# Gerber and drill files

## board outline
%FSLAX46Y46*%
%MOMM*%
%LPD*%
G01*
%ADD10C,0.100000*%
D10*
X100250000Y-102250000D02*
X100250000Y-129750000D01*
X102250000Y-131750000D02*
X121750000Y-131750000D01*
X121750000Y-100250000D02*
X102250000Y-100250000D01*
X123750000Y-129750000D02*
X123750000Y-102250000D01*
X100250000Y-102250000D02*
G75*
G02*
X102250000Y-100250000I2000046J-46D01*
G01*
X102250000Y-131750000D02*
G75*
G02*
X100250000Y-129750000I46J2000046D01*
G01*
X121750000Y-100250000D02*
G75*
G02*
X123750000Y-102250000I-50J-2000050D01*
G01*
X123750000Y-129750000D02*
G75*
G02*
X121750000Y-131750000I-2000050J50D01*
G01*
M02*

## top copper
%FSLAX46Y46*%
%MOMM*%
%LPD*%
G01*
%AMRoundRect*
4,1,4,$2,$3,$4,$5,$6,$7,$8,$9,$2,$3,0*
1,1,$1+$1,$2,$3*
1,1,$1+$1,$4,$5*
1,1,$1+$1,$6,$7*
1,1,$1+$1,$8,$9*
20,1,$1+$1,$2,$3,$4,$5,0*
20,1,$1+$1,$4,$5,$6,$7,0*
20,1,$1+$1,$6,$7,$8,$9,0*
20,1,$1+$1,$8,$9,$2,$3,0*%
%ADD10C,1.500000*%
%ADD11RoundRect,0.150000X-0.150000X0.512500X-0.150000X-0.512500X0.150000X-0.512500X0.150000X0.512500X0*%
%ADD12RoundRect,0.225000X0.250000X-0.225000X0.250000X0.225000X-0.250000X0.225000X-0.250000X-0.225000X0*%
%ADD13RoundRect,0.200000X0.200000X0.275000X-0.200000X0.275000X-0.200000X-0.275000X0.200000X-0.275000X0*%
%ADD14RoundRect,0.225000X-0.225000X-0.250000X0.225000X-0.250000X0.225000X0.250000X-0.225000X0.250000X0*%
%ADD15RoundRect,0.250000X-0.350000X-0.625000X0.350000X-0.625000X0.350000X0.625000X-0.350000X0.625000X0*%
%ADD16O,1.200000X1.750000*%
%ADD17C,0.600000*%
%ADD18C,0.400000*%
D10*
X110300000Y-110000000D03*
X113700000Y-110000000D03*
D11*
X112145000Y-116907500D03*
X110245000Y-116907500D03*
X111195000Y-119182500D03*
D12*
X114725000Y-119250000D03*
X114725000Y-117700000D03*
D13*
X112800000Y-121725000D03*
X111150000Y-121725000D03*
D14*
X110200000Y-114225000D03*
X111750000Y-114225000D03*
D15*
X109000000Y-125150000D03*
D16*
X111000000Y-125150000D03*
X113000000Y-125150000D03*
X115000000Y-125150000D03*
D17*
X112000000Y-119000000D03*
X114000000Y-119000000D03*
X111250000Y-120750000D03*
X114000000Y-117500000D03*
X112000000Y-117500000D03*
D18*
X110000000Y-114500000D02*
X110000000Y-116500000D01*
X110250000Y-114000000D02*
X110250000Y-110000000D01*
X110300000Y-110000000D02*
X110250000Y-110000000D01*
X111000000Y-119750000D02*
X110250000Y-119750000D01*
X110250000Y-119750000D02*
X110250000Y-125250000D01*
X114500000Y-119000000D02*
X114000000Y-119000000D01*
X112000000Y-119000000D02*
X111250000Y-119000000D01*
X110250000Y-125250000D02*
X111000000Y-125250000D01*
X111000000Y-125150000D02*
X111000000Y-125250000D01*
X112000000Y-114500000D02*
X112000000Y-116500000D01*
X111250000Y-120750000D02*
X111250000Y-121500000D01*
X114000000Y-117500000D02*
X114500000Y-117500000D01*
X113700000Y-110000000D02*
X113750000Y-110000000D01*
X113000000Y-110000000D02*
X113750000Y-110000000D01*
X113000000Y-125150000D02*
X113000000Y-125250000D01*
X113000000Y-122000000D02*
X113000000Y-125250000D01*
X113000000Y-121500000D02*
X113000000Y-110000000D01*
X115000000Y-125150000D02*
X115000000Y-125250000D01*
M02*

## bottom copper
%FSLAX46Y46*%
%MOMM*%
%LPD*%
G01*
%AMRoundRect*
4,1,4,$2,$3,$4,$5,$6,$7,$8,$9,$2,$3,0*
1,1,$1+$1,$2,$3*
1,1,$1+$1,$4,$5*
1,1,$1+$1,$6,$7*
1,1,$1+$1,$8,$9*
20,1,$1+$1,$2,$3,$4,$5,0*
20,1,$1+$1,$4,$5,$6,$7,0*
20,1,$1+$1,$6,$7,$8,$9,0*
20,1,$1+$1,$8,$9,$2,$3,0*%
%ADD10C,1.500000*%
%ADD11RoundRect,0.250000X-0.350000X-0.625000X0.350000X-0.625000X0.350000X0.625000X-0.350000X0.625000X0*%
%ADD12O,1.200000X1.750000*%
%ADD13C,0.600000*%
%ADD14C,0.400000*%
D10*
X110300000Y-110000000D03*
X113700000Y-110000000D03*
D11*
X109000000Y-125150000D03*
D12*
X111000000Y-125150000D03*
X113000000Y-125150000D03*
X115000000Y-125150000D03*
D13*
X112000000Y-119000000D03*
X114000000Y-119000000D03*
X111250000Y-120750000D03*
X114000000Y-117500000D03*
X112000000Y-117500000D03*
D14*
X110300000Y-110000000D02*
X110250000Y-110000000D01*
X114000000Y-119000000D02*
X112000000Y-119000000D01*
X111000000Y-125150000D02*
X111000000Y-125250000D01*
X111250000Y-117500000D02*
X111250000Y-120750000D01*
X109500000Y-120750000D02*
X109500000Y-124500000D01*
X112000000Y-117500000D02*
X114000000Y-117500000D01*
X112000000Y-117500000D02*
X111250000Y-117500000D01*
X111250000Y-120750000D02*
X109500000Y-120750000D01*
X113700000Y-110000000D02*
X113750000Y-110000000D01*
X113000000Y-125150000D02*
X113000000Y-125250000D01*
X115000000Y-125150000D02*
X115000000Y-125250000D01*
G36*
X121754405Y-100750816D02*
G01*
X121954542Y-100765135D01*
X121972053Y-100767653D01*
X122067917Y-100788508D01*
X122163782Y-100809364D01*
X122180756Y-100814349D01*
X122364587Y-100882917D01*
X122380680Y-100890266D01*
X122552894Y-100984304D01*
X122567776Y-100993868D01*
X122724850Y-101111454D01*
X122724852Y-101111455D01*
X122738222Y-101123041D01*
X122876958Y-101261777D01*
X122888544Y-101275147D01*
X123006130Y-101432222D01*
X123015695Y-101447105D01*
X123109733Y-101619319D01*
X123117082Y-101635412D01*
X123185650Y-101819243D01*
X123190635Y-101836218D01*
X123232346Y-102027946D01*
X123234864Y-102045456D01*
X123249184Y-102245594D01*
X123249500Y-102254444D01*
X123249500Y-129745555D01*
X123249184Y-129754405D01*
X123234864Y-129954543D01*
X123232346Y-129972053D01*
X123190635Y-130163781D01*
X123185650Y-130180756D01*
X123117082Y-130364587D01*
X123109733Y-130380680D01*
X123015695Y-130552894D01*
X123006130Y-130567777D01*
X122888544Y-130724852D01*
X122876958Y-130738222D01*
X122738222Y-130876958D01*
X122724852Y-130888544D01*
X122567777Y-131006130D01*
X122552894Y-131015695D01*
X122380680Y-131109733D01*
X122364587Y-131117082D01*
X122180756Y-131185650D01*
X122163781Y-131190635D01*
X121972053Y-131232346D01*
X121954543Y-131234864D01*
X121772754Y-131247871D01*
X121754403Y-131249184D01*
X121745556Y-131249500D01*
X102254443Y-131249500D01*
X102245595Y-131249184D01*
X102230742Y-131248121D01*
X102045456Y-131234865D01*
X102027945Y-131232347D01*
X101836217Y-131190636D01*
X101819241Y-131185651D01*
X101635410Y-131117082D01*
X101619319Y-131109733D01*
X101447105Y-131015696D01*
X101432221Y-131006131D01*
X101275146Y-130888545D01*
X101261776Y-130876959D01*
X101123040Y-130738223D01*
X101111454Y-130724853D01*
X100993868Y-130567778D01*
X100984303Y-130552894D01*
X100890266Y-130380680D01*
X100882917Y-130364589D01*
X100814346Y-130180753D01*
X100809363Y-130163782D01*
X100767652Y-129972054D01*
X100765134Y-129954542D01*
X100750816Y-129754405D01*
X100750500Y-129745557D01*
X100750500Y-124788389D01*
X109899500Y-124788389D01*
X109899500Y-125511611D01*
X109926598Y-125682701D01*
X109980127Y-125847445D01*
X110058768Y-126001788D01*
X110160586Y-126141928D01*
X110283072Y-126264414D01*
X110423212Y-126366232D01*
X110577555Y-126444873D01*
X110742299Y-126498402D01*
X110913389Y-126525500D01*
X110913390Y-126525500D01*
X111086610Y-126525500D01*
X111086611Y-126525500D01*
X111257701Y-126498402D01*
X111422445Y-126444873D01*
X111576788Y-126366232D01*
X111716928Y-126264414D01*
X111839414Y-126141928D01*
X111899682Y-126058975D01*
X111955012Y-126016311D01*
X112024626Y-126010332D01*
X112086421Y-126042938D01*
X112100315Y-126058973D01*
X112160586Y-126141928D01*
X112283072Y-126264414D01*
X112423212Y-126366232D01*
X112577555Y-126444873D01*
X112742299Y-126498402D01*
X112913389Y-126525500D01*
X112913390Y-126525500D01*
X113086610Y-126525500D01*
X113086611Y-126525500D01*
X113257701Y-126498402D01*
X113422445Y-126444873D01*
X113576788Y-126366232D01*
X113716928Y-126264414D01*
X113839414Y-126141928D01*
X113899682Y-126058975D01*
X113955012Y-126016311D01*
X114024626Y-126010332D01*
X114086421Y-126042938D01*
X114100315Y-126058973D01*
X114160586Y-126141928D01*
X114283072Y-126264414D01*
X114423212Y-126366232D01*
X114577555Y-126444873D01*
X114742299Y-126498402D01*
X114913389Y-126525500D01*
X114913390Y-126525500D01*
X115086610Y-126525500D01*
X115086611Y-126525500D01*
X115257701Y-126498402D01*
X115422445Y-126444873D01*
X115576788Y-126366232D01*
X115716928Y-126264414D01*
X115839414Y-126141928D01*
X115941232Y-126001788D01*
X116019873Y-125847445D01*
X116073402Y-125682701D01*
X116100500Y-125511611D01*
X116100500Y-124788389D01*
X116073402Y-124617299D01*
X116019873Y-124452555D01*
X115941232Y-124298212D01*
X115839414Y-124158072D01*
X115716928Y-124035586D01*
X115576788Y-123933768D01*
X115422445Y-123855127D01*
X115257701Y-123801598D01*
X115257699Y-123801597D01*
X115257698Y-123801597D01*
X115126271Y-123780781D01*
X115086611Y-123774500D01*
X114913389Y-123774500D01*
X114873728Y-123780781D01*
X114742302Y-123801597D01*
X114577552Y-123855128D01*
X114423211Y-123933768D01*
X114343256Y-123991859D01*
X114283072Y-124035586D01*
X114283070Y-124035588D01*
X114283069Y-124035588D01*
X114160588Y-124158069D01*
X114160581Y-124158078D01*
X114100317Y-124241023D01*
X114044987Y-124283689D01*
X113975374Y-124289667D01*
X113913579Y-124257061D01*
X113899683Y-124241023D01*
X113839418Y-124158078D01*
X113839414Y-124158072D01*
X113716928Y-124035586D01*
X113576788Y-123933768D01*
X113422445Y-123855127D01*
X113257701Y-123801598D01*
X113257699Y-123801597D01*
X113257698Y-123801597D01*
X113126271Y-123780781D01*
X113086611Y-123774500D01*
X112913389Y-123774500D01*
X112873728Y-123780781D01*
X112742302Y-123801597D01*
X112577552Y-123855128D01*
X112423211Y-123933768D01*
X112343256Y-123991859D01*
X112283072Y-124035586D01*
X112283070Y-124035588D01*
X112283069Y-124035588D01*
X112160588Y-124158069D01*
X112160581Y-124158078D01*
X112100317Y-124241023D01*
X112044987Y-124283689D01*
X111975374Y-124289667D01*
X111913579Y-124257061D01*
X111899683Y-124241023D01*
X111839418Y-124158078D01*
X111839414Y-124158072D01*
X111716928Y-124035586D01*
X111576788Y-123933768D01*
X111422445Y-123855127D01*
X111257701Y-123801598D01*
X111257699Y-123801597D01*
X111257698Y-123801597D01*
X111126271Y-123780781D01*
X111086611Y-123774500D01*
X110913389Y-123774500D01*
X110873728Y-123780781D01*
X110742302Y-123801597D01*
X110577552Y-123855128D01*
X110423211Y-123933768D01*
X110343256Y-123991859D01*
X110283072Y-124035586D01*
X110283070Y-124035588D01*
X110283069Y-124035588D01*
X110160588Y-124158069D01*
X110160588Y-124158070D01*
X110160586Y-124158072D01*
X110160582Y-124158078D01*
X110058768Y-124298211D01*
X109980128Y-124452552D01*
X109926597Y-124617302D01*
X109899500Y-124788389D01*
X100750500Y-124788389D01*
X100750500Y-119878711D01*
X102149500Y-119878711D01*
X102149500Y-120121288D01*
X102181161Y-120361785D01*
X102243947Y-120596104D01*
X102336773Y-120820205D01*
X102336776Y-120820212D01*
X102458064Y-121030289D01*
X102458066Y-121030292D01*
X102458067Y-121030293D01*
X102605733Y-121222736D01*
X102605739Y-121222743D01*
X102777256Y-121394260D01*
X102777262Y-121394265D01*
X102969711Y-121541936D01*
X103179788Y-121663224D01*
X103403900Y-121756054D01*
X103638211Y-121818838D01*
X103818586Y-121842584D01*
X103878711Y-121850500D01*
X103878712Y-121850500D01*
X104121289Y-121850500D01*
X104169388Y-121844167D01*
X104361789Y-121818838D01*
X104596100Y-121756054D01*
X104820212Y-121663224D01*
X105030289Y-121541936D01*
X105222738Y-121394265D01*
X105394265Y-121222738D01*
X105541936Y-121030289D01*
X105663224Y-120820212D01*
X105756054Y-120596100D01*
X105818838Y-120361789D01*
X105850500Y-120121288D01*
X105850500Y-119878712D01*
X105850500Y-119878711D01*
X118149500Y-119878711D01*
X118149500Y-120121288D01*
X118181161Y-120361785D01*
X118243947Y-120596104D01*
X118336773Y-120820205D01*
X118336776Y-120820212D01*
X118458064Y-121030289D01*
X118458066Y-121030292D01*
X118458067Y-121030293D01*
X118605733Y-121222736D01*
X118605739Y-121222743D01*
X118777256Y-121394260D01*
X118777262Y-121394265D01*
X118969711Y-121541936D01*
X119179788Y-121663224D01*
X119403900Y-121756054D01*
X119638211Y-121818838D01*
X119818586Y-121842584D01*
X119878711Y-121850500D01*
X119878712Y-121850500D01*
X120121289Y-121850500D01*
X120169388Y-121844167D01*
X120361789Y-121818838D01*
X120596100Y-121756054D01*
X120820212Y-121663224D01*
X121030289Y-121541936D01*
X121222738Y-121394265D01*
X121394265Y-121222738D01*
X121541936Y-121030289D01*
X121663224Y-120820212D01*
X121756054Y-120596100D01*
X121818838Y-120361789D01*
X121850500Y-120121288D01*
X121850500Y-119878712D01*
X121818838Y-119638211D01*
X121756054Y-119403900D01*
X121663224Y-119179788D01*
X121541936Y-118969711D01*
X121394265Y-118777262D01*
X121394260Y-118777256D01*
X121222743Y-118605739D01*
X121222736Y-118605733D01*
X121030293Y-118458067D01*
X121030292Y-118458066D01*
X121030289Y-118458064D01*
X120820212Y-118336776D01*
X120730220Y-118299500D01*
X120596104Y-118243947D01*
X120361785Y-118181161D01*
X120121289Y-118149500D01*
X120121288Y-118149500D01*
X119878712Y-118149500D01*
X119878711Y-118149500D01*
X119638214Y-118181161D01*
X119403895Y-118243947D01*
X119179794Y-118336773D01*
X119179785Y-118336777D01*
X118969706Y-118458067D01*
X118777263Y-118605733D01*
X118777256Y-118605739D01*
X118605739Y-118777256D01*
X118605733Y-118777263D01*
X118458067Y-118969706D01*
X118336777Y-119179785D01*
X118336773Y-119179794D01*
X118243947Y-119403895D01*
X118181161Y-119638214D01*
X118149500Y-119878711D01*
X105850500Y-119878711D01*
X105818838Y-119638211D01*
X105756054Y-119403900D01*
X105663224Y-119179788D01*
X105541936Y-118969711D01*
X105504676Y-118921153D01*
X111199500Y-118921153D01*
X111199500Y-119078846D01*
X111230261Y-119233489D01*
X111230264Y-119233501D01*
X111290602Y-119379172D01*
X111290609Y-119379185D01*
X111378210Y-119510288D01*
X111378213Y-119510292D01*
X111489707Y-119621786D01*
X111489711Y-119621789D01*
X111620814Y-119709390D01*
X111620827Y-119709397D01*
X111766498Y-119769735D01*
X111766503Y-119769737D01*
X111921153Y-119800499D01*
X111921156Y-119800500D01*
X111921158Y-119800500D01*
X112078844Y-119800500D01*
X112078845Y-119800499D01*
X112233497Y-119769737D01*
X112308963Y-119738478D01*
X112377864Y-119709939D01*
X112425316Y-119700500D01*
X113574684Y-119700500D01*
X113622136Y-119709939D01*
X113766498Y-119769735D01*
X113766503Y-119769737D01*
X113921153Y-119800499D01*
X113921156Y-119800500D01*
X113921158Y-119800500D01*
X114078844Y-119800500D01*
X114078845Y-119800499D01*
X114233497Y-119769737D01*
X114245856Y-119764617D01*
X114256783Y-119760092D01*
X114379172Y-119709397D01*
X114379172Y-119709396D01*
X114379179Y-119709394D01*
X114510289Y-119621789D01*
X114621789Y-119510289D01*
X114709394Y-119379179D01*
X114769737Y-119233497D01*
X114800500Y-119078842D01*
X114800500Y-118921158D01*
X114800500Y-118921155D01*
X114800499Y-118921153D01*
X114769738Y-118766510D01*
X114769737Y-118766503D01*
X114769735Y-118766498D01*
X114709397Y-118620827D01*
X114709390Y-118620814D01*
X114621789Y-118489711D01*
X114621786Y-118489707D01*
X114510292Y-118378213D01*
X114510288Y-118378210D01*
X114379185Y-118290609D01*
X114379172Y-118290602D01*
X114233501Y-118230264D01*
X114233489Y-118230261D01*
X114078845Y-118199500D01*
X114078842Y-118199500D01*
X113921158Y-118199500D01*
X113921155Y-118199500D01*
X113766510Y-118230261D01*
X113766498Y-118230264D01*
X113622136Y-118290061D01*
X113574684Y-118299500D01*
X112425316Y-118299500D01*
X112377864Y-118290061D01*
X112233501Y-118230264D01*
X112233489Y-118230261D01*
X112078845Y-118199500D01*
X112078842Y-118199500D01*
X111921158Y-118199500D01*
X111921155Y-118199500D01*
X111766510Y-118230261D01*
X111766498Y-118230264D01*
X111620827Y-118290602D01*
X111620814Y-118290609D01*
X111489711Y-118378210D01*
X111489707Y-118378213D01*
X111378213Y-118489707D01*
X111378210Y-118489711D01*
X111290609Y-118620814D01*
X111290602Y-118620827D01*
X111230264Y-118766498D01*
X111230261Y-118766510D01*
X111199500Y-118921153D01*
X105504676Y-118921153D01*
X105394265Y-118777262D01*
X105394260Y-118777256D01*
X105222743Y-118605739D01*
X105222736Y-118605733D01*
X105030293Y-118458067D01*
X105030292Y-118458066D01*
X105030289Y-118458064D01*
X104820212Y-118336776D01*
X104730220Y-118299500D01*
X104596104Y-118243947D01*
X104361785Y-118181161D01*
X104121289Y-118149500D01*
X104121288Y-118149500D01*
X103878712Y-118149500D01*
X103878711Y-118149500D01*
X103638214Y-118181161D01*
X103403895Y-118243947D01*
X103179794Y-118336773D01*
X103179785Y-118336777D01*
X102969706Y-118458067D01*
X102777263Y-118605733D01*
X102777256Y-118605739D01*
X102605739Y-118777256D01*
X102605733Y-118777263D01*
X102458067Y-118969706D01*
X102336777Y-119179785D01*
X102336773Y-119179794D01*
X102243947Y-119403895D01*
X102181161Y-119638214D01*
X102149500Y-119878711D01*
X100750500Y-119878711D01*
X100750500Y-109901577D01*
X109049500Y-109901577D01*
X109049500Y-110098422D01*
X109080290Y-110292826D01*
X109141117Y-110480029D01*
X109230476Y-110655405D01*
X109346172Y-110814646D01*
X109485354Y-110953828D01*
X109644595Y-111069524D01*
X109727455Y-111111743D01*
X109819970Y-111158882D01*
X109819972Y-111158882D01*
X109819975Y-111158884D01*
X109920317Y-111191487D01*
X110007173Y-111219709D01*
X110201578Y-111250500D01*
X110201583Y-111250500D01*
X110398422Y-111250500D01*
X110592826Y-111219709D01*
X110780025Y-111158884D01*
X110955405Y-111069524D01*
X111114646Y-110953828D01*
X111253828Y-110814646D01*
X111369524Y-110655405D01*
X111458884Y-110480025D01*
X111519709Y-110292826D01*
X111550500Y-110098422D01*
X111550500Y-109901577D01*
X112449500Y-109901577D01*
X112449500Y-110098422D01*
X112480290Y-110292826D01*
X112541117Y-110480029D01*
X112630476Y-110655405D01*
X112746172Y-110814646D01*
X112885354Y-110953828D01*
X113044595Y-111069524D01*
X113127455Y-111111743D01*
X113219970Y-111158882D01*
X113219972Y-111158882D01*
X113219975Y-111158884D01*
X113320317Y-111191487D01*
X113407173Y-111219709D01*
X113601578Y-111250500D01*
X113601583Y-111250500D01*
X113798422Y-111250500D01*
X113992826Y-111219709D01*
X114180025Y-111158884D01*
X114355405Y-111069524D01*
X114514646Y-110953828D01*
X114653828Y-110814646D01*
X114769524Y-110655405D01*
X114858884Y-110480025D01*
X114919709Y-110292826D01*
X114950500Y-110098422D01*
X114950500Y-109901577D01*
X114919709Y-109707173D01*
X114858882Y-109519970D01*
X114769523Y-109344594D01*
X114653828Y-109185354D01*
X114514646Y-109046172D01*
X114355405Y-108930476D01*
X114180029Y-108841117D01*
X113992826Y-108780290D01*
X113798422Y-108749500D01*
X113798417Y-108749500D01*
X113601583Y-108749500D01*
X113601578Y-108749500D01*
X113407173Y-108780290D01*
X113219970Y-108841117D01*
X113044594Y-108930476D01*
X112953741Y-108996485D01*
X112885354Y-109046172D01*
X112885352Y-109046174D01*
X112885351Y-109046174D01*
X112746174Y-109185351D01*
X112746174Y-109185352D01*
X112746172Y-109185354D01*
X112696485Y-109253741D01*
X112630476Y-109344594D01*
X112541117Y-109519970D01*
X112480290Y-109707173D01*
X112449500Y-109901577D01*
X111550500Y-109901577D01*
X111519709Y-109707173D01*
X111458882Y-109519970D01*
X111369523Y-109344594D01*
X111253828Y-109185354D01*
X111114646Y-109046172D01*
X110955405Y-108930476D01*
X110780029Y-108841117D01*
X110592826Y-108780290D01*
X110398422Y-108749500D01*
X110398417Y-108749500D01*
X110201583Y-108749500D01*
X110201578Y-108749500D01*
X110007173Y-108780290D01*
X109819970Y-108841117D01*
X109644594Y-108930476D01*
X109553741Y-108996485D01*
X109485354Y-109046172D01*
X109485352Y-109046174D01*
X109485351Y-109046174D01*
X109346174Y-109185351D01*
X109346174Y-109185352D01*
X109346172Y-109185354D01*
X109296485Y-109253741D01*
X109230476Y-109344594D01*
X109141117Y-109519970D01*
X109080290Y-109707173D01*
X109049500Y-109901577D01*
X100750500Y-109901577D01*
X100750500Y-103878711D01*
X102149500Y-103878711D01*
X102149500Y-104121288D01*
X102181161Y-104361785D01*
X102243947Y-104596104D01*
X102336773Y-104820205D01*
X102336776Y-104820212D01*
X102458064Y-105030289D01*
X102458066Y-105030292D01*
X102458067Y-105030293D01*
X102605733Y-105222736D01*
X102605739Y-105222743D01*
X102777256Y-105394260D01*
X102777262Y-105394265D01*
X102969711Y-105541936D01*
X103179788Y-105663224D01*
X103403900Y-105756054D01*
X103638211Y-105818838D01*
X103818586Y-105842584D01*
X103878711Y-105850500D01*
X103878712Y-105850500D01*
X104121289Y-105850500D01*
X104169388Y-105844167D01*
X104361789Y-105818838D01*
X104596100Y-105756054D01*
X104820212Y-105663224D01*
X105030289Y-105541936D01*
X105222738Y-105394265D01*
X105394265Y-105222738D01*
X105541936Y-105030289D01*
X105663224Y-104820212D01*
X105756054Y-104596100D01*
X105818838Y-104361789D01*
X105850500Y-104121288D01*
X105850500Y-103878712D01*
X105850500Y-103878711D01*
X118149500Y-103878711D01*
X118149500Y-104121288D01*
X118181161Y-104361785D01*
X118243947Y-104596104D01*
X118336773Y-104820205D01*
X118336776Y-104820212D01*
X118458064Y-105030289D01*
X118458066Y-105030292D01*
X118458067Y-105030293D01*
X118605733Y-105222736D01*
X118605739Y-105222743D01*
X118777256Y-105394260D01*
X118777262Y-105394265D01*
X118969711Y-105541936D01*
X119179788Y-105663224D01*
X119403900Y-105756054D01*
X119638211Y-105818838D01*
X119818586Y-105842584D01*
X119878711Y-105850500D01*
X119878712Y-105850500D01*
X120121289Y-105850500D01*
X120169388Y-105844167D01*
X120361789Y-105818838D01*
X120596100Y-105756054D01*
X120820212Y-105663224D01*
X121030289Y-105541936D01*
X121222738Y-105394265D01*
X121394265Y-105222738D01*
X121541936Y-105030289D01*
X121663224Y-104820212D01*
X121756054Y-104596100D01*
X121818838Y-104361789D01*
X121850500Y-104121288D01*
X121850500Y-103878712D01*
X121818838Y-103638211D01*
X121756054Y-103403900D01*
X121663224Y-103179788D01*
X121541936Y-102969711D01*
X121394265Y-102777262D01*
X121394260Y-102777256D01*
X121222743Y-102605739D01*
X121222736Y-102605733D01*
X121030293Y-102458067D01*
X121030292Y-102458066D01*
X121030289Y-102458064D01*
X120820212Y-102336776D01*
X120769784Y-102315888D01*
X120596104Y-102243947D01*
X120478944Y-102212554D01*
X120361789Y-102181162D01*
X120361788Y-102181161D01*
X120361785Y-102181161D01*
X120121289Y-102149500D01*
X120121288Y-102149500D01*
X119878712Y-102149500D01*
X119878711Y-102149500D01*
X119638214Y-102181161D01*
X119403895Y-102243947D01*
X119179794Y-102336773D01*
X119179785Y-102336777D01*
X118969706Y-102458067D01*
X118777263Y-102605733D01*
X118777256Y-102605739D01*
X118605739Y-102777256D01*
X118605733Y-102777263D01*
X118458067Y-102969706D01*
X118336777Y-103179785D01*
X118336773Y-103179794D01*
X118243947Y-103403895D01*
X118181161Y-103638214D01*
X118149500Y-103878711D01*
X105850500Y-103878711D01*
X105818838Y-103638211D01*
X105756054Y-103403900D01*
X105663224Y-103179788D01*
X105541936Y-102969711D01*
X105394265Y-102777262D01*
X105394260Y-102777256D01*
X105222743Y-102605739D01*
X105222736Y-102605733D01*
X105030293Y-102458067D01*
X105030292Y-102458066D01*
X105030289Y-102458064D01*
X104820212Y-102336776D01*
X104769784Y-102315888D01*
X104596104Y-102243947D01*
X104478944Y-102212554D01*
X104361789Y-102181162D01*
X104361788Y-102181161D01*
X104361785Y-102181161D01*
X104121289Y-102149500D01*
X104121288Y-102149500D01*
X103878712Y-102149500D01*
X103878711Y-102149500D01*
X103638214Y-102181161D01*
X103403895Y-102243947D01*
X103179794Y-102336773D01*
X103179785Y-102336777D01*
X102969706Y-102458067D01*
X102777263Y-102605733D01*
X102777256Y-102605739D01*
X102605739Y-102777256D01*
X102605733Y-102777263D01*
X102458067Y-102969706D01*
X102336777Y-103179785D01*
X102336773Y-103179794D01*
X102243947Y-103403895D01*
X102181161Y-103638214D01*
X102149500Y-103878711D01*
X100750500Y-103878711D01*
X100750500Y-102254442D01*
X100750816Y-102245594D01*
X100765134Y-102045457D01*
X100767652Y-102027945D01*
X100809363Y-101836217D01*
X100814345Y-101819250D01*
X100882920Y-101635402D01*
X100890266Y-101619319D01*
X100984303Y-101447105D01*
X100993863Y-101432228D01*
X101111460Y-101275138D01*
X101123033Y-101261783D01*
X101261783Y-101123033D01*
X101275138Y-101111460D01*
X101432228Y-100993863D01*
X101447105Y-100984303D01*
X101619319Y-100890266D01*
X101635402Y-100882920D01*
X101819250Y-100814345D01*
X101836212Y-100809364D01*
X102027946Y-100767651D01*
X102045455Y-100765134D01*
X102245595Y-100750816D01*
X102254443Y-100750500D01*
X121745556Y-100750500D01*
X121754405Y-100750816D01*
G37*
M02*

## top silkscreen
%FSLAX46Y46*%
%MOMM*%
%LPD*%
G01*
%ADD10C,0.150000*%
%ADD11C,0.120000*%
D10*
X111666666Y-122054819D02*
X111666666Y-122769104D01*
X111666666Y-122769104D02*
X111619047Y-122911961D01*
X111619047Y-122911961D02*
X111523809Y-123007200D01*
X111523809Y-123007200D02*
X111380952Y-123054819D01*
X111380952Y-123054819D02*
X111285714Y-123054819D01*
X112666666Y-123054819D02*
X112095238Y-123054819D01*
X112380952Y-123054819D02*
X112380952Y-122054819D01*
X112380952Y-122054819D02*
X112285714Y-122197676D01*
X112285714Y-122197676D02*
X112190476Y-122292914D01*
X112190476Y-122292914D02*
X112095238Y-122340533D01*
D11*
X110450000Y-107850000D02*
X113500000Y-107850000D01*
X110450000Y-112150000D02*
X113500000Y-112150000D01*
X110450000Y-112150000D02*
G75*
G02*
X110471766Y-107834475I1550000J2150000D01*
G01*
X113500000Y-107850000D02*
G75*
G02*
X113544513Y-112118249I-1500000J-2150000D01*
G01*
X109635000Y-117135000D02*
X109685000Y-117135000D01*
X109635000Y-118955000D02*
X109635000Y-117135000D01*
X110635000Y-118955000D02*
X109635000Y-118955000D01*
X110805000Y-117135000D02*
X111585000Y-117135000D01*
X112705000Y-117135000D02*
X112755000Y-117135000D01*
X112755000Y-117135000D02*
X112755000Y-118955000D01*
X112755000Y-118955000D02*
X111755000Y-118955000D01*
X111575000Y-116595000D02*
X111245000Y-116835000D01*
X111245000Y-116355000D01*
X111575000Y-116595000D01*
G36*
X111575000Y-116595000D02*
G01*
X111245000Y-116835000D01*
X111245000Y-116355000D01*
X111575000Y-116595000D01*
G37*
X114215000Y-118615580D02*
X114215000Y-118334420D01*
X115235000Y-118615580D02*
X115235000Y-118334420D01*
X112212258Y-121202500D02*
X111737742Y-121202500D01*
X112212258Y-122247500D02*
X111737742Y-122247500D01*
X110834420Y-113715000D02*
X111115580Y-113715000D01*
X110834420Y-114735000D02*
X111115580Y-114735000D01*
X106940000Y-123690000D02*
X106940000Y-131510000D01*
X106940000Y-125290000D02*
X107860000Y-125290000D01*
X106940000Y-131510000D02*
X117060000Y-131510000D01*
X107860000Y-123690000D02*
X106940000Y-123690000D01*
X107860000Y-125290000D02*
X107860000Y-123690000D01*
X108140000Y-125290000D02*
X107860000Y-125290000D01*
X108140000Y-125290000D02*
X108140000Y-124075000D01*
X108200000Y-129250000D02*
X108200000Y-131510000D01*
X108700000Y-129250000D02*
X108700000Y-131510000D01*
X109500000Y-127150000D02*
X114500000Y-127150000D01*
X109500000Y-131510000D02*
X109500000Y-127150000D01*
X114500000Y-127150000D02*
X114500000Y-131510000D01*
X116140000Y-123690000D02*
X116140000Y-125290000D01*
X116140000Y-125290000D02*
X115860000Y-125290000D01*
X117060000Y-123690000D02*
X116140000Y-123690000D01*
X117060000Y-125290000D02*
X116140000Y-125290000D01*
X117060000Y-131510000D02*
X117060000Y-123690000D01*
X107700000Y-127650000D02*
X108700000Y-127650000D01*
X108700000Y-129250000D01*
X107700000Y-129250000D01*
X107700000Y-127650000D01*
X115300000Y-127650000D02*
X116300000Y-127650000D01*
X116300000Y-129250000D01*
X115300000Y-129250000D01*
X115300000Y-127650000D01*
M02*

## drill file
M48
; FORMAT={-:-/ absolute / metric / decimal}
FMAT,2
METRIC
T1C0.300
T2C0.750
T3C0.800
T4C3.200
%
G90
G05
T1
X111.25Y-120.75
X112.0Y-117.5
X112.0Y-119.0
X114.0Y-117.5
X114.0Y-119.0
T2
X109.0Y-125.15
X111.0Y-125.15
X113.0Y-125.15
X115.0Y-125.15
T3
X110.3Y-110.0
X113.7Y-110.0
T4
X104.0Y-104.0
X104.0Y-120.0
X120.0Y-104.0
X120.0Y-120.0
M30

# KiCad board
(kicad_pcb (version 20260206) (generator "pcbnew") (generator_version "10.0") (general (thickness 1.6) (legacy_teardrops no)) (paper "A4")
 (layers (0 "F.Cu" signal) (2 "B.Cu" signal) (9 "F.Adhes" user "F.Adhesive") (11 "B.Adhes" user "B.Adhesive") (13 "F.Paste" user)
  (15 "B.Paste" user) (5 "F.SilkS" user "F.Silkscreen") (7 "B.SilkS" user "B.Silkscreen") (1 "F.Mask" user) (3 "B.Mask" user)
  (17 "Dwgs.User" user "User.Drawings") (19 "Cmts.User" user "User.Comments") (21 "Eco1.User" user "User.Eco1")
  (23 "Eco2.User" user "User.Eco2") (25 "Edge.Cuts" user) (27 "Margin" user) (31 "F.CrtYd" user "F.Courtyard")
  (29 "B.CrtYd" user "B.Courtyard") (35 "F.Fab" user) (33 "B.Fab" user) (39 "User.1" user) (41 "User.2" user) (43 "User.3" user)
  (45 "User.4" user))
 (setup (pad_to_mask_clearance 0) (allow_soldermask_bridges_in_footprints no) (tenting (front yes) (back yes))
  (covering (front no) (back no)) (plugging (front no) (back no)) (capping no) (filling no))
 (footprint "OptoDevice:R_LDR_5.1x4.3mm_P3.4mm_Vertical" (layer "F.Cu") (at 110.3 110)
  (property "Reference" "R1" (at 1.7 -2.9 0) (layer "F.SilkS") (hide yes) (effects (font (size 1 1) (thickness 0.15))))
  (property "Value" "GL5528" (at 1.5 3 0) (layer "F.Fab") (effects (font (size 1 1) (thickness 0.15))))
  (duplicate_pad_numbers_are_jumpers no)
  (fp_line (start 0.15 -2.15) (end 3.2 -2.15) (stroke (width 0.12) (type solid)) (layer "F.SilkS"))
  (fp_line (start 0.15 2.15) (end 3.2 2.15) (stroke (width 0.12) (type solid)) (layer "F.SilkS"))
  (fp_arc (start 0.15 2.15) (mid -0.950438 -0.013368) (end 0.171766 -2.165525) (stroke (width 0.12) (type solid)) (layer "F.SilkS"))
  (fp_arc (start 3.2 -2.15) (mid 4.321403 -0.027338) (end 3.244513 2.118249) (stroke (width 0.12) (type solid)) (layer "F.SilkS"))
  (pad "1" thru_hole circle (at 0 0) (size 1.5 1.5) (drill 0.8) (layers "*.Cu" "*.Mask") (remove_unused_layers no) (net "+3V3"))
  (pad "2" thru_hole circle (at 3.4 0) (size 1.5 1.5) (drill 0.8) (layers "*.Cu" "*.Mask") (remove_unused_layers no) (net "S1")))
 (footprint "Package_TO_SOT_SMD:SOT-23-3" (layer "F.Cu") (at 111.195 118.045 -90)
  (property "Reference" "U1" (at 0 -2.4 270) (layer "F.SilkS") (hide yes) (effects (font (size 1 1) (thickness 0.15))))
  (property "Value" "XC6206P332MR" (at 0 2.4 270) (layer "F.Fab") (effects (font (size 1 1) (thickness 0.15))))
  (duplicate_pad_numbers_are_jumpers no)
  (fp_line (start -0.91 1.56) (end -0.91 1.51) (stroke (width 0.12) (type solid)) (layer "F.SilkS"))
  (fp_line (start 0.91 1.56) (end -0.91 1.56) (stroke (width 0.12) (type solid)) (layer "F.SilkS"))
  (fp_line (start 0.91 0.56) (end 0.91 1.56) (stroke (width 0.12) (type solid)) (layer "F.SilkS"))
  (fp_line (start -0.91 0.39) (end -0.91 -0.39) (stroke (width 0.12) (type solid)) (layer "F.SilkS"))
  (fp_line (start -0.91 -1.51) (end -0.91 -1.56) (stroke (width 0.12) (type solid)) (layer "F.SilkS"))
  (fp_line (start -0.91 -1.56) (end 0.91 -1.56) (stroke (width 0.12) (type solid)) (layer "F.SilkS"))
  (fp_line (start 0.91 -1.56) (end 0.91 -0.56) (stroke (width 0.12) (type solid)) (layer "F.SilkS"))
  (fp_poly (pts (xy -1.45 -0.38) (xy -1.21 -0.05) (xy -1.69 -0.05)) (stroke (width 0.12) (type solid)) (fill yes) (layer "F.SilkS"))
  (pad "1" smd roundrect (at -1.1375 -0.95 270) (size 1.325 0.6) (layers "F.Cu" "F.Mask" "F.Paste") (roundrect_rratio 0.25) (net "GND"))
  (pad "2" smd roundrect (at -1.1375 0.95 270) (size 1.325 0.6) (layers "F.Cu" "F.Mask" "F.Paste") (roundrect_rratio 0.25) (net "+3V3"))
  (pad "3" smd roundrect (at 1.1375 0 270) (size 1.325 0.6) (layers "F.Cu" "F.Mask" "F.Paste") (roundrect_rratio 0.25) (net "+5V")))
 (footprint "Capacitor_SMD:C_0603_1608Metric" (layer "F.Cu") (at 114.725 118.475 90)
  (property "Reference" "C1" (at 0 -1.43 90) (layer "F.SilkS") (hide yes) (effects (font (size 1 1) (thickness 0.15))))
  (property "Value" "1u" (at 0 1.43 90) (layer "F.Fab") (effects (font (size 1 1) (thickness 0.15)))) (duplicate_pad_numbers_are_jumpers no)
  (fp_line (start -0.14058 -0.51) (end 0.14058 -0.51) (stroke (width 0.12) (type solid)) (layer "F.SilkS"))
  (fp_line (start -0.14058 0.51) (end 0.14058 0.51) (stroke (width 0.12) (type solid)) (layer "F.SilkS"))
  (pad "1" smd roundrect (at -0.775 0 90) (size 0.9 0.95) (layers "F.Cu" "F.Mask" "F.Paste") (roundrect_rratio 0.25) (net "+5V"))
  (pad "2" smd roundrect (at 0.775 0 90) (size 0.9 0.95) (layers "F.Cu" "F.Mask" "F.Paste") (roundrect_rratio 0.25) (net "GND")))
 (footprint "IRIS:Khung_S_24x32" (layer "F.Cu") (at 100 132)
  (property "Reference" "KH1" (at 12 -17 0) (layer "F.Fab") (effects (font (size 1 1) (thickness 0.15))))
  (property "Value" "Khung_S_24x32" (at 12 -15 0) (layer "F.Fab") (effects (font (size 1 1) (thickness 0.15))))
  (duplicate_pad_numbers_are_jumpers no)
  (fp_line (start 0.25 -29.75) (end 0.25 -2.25) (stroke (width 0.1) (type solid)) (layer "Edge.Cuts"))
  (fp_line (start 2.25 -0.25) (end 21.75 -0.25) (stroke (width 0.1) (type solid)) (layer "Edge.Cuts"))
  (fp_line (start 21.75 -31.75) (end 2.25 -31.75) (stroke (width 0.1) (type solid)) (layer "Edge.Cuts"))
  (fp_line (start 23.75 -2.25) (end 23.75 -29.75) (stroke (width 0.1) (type solid)) (layer "Edge.Cuts"))
  (fp_arc (start 0.25 -29.75) (mid 0.8358 -31.1642) (end 2.25 -31.75) (stroke (width 0.1) (type solid)) (layer "Edge.Cuts"))
  (fp_arc (start 2.25 -0.25) (mid 0.8358 -0.8358) (end 0.25 -2.25) (stroke (width 0.1) (type solid)) (layer "Edge.Cuts"))
  (fp_arc (start 21.75 -31.75) (mid 23.164199 -31.164199) (end 23.75 -29.75) (stroke (width 0.1) (type solid)) (layer "Edge.Cuts"))
  (fp_arc (start 23.75 -2.25) (mid 23.164199 -0.835801) (end 21.75 -0.25) (stroke (width 0.1) (type solid)) (layer "Edge.Cuts"))
  (pad "" np_thru_hole circle (at 4 -28) (size 3.2 3.2) (drill 3.2) (layers "*.Cu" "*.Mask"))
  (pad "" np_thru_hole circle (at 4 -12) (size 3.2 3.2) (drill 3.2) (layers "*.Cu" "*.Mask"))
  (pad "" np_thru_hole circle (at 20 -28) (size 3.2 3.2) (drill 3.2) (layers "*.Cu" "*.Mask"))
  (pad "" np_thru_hole circle (at 20 -12) (size 3.2 3.2) (drill 3.2) (layers "*.Cu" "*.Mask")))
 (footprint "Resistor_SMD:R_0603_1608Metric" (layer "F.Cu") (at 111.975 121.725 180)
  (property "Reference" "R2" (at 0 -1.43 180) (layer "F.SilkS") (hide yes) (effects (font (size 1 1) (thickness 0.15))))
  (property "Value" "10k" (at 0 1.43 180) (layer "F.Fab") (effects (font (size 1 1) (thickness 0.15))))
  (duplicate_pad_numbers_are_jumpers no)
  (fp_line (start -0.237258 0.5225) (end 0.237258 0.5225) (stroke (width 0.12) (type solid)) (layer "F.SilkS"))
  (fp_line (start -0.237258 -0.5225) (end 0.237258 -0.5225) (stroke (width 0.12) (type solid)) (layer "F.SilkS"))
  (pad "1" smd roundrect (at -0.825 0 180) (size 0.8 0.95) (layers "F.Cu" "F.Mask" "F.Paste") (roundrect_rratio 0.25) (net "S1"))
  (pad "2" smd roundrect (at 0.825 0 180) (size 0.8 0.95) (layers "F.Cu" "F.Mask" "F.Paste") (roundrect_rratio 0.25) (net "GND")))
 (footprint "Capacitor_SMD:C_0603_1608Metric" (layer "F.Cu") (at 110.975 114.225)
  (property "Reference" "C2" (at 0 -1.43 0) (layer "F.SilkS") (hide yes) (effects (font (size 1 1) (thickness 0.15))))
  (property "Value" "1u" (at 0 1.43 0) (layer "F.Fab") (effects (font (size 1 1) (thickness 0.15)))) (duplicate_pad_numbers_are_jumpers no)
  (fp_line (start -0.14058 -0.51) (end 0.14058 -0.51) (stroke (width 0.12) (type solid)) (layer "F.SilkS"))
  (fp_line (start -0.14058 0.51) (end 0.14058 0.51) (stroke (width 0.12) (type solid)) (layer "F.SilkS"))
  (pad "1" smd roundrect (at -0.775 0) (size 0.9 0.95) (layers "F.Cu" "F.Mask" "F.Paste") (roundrect_rratio 0.25) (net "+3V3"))
  (pad "2" smd roundrect (at 0.775 0) (size 0.9 0.95) (layers "F.Cu" "F.Mask" "F.Paste") (roundrect_rratio 0.25) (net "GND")))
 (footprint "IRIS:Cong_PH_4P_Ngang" (layer "F.Cu") (at 109 125.15)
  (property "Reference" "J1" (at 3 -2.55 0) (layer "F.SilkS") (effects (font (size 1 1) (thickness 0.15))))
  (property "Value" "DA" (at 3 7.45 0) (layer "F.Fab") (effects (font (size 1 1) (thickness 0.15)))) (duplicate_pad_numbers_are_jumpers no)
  (fp_line (start -2.06 -1.46) (end -2.06 6.36) (stroke (width 0.12) (type solid)) (layer "F.SilkS"))
  (fp_line (start -2.06 0.14) (end -1.14 0.14) (stroke (width 0.12) (type solid)) (layer "F.SilkS"))
  (fp_line (start -2.06 6.36) (end 8.06 6.36) (stroke (width 0.12) (type solid)) (layer "F.SilkS"))
  (fp_line (start -1.14 -1.46) (end -2.06 -1.46) (stroke (width 0.12) (type solid)) (layer "F.SilkS"))
  (fp_line (start -1.14 0.14) (end -1.14 -1.46) (stroke (width 0.12) (type solid)) (layer "F.SilkS"))
  (fp_line (start -0.86 0.14) (end -1.14 0.14) (stroke (width 0.12) (type solid)) (layer "F.SilkS"))
  (fp_line (start -0.86 0.14) (end -0.86 -1.075) (stroke (width 0.12) (type solid)) (layer "F.SilkS"))
  (fp_line (start -0.8 4.1) (end -0.8 6.36) (stroke (width 0.12) (type solid)) (layer "F.SilkS"))
  (fp_line (start -0.3 4.1) (end -0.3 6.36) (stroke (width 0.12) (type solid)) (layer "F.SilkS"))
  (fp_line (start 0.5 2) (end 5.5 2) (stroke (width 0.12) (type solid)) (layer "F.SilkS"))
  (fp_line (start 0.5 6.36) (end 0.5 2) (stroke (width 0.12) (type solid)) (layer "F.SilkS"))
  (fp_line (start 5.5 2) (end 5.5 6.36) (stroke (width 0.12) (type solid)) (layer "F.SilkS"))
  (fp_line (start 7.14 -1.46) (end 7.14 0.14) (stroke (width 0.12) (type solid)) (layer "F.SilkS"))
  (fp_line (start 7.14 0.14) (end 6.86 0.14) (stroke (width 0.12) (type solid)) (layer "F.SilkS"))
  (fp_line (start 8.06 -1.46) (end 7.14 -1.46) (stroke (width 0.12) (type solid)) (layer "F.SilkS"))
  (fp_line (start 8.06 0.14) (end 7.14 0.14) (stroke (width 0.12) (type solid)) (layer "F.SilkS"))
  (fp_line (start 8.06 6.36) (end 8.06 -1.46) (stroke (width 0.12) (type solid)) (layer "F.SilkS"))
  (fp_rect (start -1.3 2.5) (end -0.3 4.1) (stroke (width 0.12) (type solid)) (fill no) (layer "F.SilkS"))
  (fp_rect (start 6.3 2.5) (end 7.3 4.1) (stroke (width 0.12) (type solid)) (fill no) (layer "F.SilkS"))
  (pad "1" thru_hole roundrect (at 0 0) (size 1.2 1.75) (drill 0.75) (layers "*.Cu" "*.Mask") (remove_unused_layers no)
   (roundrect_rratio 0.208333) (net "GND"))
  (pad "2" thru_hole oval (at 2 0) (size 1.2 1.75) (drill 0.75) (layers "*.Cu" "*.Mask") (remove_unused_layers no) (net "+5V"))
  (pad "3" thru_hole oval (at 4 0) (size 1.2 1.75) (drill 0.75) (layers "*.Cu" "*.Mask") (remove_unused_layers no) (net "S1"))
  (pad "4" thru_hole oval (at 6 0) (size 1.2 1.75) (drill 0.75) (layers "*.Cu" "*.Mask") (remove_unused_layers no)
   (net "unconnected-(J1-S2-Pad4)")))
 (segment (start 110 114.5) (end 110 116.5) (width 0.4) (layer "F.Cu") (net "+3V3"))
 (segment (start 110.25 114) (end 110.25 110) (width 0.4) (layer "F.Cu") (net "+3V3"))
 (segment (start 110.3 110) (end 110.25 110) (width 0.4) (layer "F.Cu") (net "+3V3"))
 (segment (start 110.3 110) (end 110.25 110) (width 0.4) (layer "B.Cu") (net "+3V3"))
 (segment (start 111 119.75) (end 110.25 119.75) (width 0.4) (layer "F.Cu") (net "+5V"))
 (segment (start 110.25 119.75) (end 110.25 125.25) (width 0.4) (layer "F.Cu") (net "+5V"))
 (segment (start 114.5 119) (end 114 119) (width 0.4) (layer "F.Cu") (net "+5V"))
 (segment (start 112 119) (end 111.25 119) (width 0.4) (layer "F.Cu") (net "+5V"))
 (segment (start 110.25 125.25) (end 111 125.25) (width 0.4) (layer "F.Cu") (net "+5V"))
 (segment (start 111 125.15) (end 111 125.25) (width 0.4) (layer "F.Cu") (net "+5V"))
 (via (at 112 119) (size 0.6) (drill 0.3) (layers "F.Cu" "B.Cu") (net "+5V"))
 (via (at 114 119) (size 0.6) (drill 0.3) (layers "F.Cu" "B.Cu") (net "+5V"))
 (segment (start 114 119) (end 112 119) (width 0.4) (layer "B.Cu") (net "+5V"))
 (segment (start 111 125.15) (end 111 125.25) (width 0.4) (layer "B.Cu") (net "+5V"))
 (segment (start 112 114.5) (end 112 116.5) (width 0.4) (layer "F.Cu") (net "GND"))
 (segment (start 111.25 120.75) (end 111.25 121.5) (width 0.4) (layer "F.Cu") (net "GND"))
 (segment (start 114 117.5) (end 114.5 117.5) (width 0.4) (layer "F.Cu") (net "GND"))
 (via (at 111.25 120.75) (size 0.6) (drill 0.3) (layers "F.Cu" "B.Cu") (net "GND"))
 (via (at 114 117.5) (size 0.6) (drill 0.3) (layers "F.Cu" "B.Cu") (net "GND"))
 (via (at 112 117.5) (size 0.6) (drill 0.3) (layers "F.Cu" "B.Cu") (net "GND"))
 (segment (start 111.25 117.5) (end 111.25 120.75) (width 0.4) (layer "B.Cu") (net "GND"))
 (segment (start 109.5 120.75) (end 109.5 124.5) (width 0.4) (layer "B.Cu") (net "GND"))
 (segment (start 112 117.5) (end 114 117.5) (width 0.4) (layer "B.Cu") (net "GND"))
 (segment (start 112 117.5) (end 111.25 117.5) (width 0.4) (layer "B.Cu") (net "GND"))
 (segment (start 111.25 120.75) (end 109.5 120.75) (width 0.4) (layer "B.Cu") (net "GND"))
 (segment (start 113.7 110) (end 113.75 110) (width 0.4) (layer "F.Cu") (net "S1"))
 (segment (start 113 110) (end 113.75 110) (width 0.4) (layer "F.Cu") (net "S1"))
 (segment (start 113 125.15) (end 113 125.25) (width 0.4) (layer "F.Cu") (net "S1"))
 (segment (start 113 122) (end 113 125.25) (width 0.4) (layer "F.Cu") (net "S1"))
 (segment (start 113 121.5) (end 113 110) (width 0.4) (layer "F.Cu") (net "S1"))
 (segment (start 113.7 110) (end 113.75 110) (width 0.4) (layer "B.Cu") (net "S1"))
 (segment (start 113 125.15) (end 113 125.25) (width 0.4) (layer "B.Cu") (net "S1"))
 (segment (start 115 125.15) (end 115 125.25) (width 0.4) (layer "F.Cu") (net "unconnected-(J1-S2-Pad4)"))
 (segment (start 115 125.15) (end 115 125.25) (width 0.4) (layer "B.Cu") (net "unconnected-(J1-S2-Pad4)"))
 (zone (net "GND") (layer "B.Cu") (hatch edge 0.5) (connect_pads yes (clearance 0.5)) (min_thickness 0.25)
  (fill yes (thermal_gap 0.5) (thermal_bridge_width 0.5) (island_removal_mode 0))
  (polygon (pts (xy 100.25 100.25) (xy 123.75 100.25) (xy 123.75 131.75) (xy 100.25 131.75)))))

